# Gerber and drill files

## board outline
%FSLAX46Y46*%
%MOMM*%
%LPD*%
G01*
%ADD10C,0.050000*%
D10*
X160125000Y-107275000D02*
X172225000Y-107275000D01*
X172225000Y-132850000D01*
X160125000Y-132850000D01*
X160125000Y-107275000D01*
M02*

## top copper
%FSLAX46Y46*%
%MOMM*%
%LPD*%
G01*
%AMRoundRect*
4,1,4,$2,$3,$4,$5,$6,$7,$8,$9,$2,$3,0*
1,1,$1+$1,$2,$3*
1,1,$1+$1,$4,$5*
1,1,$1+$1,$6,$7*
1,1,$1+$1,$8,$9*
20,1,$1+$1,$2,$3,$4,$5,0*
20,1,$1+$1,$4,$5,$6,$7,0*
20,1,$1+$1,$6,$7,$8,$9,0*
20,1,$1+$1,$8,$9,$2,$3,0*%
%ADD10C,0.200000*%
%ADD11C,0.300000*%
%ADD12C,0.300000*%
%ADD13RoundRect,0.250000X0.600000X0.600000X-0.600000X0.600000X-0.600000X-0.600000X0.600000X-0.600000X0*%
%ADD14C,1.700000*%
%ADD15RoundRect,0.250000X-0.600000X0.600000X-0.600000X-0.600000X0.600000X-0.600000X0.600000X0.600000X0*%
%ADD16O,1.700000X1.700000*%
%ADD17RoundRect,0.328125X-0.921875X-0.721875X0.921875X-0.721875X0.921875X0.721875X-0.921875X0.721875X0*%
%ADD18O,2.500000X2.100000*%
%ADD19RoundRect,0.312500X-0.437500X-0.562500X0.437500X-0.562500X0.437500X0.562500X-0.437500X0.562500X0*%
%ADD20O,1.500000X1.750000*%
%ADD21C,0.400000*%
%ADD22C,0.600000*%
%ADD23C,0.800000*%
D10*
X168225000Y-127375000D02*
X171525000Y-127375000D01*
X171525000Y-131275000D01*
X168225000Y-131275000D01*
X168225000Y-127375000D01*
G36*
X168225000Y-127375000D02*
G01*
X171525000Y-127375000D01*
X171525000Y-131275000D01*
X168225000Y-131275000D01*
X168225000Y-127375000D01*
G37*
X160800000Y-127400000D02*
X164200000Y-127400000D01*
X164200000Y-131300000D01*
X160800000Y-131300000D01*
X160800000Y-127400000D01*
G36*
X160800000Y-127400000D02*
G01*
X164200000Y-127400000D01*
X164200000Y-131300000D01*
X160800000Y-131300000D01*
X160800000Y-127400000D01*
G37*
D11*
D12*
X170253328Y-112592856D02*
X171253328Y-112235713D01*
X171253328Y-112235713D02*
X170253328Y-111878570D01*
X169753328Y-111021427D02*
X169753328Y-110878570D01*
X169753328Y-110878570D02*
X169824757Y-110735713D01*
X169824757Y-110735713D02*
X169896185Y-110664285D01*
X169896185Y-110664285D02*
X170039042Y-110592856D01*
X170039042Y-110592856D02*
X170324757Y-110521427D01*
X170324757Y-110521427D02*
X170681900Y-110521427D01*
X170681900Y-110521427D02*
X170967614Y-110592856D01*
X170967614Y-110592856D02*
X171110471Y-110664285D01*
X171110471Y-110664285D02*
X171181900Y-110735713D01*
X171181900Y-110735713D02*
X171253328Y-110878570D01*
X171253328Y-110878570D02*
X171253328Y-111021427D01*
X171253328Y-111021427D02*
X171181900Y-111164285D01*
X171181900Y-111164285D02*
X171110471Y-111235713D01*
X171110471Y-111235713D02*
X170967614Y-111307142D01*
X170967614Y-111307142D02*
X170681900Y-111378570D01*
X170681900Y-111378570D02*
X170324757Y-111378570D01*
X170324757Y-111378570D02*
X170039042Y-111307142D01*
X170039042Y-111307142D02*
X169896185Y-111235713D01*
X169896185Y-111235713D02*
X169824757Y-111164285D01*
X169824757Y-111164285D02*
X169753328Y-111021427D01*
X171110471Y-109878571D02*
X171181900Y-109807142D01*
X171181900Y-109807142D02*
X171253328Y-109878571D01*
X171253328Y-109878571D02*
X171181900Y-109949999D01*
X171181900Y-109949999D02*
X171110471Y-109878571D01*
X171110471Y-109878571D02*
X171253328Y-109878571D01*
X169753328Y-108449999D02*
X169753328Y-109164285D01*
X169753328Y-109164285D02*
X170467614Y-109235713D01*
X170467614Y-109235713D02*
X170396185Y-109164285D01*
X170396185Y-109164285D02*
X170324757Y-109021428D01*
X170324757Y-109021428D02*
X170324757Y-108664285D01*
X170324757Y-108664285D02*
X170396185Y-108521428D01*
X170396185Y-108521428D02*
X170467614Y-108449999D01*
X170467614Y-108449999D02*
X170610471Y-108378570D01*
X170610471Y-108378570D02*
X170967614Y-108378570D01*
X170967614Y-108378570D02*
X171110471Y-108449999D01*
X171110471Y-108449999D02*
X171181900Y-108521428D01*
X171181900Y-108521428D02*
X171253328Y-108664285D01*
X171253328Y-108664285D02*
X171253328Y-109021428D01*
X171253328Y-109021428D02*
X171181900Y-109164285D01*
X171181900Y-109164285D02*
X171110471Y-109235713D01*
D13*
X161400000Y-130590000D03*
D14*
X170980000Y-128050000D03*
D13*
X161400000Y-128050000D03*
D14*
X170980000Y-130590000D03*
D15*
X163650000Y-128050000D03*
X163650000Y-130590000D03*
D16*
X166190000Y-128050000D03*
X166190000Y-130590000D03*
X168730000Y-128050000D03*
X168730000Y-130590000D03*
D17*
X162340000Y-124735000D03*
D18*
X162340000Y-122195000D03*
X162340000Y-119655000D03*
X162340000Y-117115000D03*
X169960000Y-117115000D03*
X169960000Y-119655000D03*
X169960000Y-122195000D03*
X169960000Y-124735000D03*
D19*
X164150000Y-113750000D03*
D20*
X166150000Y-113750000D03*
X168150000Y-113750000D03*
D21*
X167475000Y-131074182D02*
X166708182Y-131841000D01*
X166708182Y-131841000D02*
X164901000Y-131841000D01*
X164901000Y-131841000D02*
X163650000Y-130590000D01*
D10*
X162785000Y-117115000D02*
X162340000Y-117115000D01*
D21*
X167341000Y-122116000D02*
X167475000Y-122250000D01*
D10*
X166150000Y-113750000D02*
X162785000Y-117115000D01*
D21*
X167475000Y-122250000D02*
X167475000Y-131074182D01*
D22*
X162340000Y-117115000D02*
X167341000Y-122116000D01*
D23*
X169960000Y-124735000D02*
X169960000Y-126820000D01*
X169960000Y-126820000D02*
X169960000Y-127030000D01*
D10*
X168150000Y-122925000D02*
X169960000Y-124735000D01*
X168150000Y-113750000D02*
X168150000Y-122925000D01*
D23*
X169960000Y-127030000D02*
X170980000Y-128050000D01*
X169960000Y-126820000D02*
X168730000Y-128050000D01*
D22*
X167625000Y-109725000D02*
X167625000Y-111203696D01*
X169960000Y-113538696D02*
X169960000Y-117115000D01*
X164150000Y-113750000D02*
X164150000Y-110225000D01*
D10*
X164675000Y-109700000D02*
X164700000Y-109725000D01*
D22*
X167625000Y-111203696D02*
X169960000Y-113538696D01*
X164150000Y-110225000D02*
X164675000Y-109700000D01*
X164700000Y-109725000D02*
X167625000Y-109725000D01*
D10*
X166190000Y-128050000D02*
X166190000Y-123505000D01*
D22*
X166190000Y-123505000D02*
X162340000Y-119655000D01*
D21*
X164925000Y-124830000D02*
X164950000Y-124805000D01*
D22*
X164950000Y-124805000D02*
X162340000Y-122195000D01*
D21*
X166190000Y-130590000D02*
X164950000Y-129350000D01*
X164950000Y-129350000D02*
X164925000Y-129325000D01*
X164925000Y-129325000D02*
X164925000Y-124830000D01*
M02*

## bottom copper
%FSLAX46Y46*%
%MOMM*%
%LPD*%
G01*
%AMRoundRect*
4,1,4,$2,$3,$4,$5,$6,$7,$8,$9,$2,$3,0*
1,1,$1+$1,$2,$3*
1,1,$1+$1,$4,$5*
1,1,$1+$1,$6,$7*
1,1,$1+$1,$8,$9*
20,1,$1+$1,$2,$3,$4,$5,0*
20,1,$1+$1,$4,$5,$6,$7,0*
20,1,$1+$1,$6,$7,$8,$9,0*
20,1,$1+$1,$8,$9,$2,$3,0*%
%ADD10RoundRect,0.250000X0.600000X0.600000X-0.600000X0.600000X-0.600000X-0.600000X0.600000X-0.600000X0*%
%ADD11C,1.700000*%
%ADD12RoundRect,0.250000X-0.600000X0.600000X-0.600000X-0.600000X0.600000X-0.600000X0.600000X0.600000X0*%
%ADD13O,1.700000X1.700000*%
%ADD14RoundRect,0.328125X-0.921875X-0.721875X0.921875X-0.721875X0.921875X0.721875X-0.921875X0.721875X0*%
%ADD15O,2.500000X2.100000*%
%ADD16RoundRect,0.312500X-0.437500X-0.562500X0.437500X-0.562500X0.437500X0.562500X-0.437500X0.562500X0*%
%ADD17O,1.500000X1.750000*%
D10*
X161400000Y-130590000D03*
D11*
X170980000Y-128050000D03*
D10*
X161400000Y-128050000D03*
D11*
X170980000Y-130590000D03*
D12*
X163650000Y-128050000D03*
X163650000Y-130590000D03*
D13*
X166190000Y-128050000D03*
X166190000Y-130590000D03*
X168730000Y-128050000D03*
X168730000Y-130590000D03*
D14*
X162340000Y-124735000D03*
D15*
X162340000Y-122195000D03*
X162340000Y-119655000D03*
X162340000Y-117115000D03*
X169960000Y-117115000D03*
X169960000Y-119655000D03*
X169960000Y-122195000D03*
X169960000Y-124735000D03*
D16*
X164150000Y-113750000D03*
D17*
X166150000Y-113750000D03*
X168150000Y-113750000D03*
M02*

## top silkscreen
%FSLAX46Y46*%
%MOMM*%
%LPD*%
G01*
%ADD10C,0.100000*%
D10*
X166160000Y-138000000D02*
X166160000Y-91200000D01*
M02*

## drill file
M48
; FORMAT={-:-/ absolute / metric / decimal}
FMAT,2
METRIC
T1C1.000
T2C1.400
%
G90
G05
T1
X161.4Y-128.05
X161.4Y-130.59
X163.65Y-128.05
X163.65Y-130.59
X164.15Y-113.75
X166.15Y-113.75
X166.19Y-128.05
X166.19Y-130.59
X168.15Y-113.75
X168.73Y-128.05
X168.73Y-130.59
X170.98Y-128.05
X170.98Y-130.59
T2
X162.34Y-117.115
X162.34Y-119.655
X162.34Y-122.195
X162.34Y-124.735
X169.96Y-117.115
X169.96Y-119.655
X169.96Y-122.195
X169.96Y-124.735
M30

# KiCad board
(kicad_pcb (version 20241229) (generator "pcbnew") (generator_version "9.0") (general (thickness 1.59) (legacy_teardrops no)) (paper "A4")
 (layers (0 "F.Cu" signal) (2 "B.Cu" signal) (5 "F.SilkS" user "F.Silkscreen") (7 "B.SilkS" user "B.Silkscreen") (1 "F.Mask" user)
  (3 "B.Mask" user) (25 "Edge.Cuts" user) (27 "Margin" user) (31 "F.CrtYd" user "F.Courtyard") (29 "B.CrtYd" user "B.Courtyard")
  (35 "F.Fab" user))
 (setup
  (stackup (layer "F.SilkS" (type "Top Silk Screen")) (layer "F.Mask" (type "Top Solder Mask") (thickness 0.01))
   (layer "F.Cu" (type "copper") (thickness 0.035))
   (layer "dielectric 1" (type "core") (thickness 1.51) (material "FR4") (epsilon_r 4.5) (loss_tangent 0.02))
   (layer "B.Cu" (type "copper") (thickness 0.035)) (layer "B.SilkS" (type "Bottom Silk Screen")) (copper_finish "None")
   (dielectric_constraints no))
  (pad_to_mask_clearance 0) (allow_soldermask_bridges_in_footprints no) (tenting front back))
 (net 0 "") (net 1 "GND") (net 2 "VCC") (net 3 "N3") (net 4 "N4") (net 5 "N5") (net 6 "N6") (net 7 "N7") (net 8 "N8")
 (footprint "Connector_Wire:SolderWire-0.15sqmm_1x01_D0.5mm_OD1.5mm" (layer "F.Cu") (at 161.4 130.59 180)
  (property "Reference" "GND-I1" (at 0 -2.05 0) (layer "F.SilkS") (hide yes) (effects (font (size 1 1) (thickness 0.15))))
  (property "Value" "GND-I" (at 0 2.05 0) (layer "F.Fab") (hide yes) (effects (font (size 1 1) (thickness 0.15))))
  (pad "1" thru_hole roundrect (at 0 0 180) (size 1.7 1.7) (drill 1) (layers "*.Cu" "*.Mask") (remove_unused_layers no)
   (roundrect_rratio 0.147059) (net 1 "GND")))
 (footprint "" (layer "F.Cu") (at 170.98 128.05)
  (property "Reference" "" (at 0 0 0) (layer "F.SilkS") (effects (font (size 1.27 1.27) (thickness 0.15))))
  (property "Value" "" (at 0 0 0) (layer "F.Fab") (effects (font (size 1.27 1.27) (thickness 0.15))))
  (pad "1" thru_hole circle (at 0 0) (size 1.7 1.7) (drill 1) (layers "*.Cu" "*.Mask") (remove_unused_layers no) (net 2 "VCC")))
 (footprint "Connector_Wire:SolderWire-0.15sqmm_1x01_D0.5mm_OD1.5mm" (layer "F.Cu") (at 161.4 128.05 180)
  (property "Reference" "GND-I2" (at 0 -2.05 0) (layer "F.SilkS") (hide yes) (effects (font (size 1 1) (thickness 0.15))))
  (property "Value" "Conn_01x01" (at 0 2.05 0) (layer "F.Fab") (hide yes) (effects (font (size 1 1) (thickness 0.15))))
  (pad "1" thru_hole roundrect (at 0 0 180) (size 1.7 1.7) (drill 1) (layers "*.Cu" "*.Mask") (remove_unused_layers no)
   (roundrect_rratio 0.147059) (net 1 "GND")))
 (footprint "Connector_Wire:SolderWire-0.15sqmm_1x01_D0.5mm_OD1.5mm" (layer "B.Cu") (at 170.98 130.59)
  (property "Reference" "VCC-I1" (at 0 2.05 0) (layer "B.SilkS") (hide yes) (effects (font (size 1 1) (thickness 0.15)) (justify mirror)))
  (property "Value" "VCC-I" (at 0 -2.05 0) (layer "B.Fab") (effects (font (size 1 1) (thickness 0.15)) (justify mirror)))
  (pad "1" thru_hole circle (at 0 0) (size 1.7 1.7) (drill 1) (layers "*.Cu" "*.Mask") (remove_unused_layers no) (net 2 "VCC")))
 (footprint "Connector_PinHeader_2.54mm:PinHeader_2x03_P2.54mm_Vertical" (layer "B.Cu") (at 163.65 128.05 -90)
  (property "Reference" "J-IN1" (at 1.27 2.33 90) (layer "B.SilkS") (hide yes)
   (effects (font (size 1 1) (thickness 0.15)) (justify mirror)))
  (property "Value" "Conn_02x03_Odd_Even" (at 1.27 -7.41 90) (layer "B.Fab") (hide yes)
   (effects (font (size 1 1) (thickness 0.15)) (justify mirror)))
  (pad "1" thru_hole roundrect (at 0 0 270) (size 1.7 1.7) (drill 1) (layers "*.Cu" "*.Mask") (remove_unused_layers no)
   (roundrect_rratio 0.1470588235) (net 1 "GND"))
  (pad "2" thru_hole roundrect (at 2.54 0 270) (size 1.7 1.7) (drill 1) (layers "*.Cu" "*.Mask") (remove_unused_layers no)
   (roundrect_rratio 0.1470588235) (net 1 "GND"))
  (pad "3" thru_hole oval (at 0 -2.54 270) (size 1.7 1.7) (drill 1) (layers "*.Cu" "*.Mask") (remove_unused_layers no) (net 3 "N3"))
  (pad "4" thru_hole oval (at 2.54 -2.54 270) (size 1.7 1.7) (drill 1) (layers "*.Cu" "*.Mask") (remove_unused_layers no) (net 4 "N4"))
  (pad "5" thru_hole oval (at 0 -5.08 270) (size 1.7 1.7) (drill 1) (layers "*.Cu" "*.Mask") (remove_unused_layers no) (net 2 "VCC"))
  (pad "6" thru_hole oval (at 2.54 -5.08 270) (size 1.7 1.7) (drill 1) (layers "*.Cu" "*.Mask") (remove_unused_layers no) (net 2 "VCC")))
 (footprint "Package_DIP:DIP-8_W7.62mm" (layer "B.Cu") (at 162.34 124.735)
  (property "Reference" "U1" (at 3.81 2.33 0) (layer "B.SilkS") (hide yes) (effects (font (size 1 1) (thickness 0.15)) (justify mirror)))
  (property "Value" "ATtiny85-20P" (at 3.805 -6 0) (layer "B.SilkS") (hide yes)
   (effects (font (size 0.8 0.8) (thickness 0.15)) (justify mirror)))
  (pad "1" thru_hole roundrect (at 0 0) (size 2.5 2.1) (drill 1.4) (layers "*.Cu" "*.Mask") (remove_unused_layers no)
   (roundrect_rratio 0.15625) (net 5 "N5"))
  (pad "2" thru_hole oval (at 0 -2.54) (size 2.5 2.1) (drill 1.4) (layers "*.Cu" "*.Mask") (remove_unused_layers no) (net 4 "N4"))
  (pad "3" thru_hole oval (at 0 -5.08) (size 2.5 2.1) (drill 1.4) (layers "*.Cu" "*.Mask") (remove_unused_layers no) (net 3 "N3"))
  (pad "4" thru_hole oval (at 0 -7.62) (size 2.5 2.1) (drill 1.4) (layers "*.Cu" "*.Mask") (remove_unused_layers no) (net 1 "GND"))
  (pad "5" thru_hole oval (at 7.62 -7.62) (size 2.5 2.1) (drill 1.4) (layers "*.Cu" "*.Mask") (remove_unused_layers no) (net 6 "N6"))
  (pad "6" thru_hole oval (at 7.62 -5.08) (size 2.5 2.1) (drill 1.4) (layers "*.Cu" "*.Mask") (remove_unused_layers no) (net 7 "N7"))
  (pad "7" thru_hole oval (at 7.62 -2.54) (size 2.5 2.1) (drill 1.4) (layers "*.Cu" "*.Mask") (remove_unused_layers no) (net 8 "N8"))
  (pad "8" thru_hole oval (at 7.62 0) (size 2.5 2.1) (drill 1.4) (layers "*.Cu" "*.Mask") (remove_unused_layers no) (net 2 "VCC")))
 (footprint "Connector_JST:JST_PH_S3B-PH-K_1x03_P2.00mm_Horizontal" (layer "B.Cu") (at 164.15 113.75)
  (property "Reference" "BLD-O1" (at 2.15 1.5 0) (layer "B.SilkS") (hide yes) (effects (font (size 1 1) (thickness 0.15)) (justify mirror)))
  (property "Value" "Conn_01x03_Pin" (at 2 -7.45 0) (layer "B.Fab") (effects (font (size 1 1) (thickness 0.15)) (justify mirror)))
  (pad "1" thru_hole roundrect (at 0 0) (size 1.5 1.75) (drill 1) (layers "*.Cu" "*.Mask") (remove_unused_layers no)
   (roundrect_rratio 0.208333) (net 6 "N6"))
  (pad "2" thru_hole oval (at 2 0) (size 1.5 1.75) (drill 1) (layers "*.Cu" "*.Mask") (remove_unused_layers no) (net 1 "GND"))
  (pad "3" thru_hole oval (at 4 0) (size 1.5 1.75) (drill 1) (layers "*.Cu" "*.Mask") (remove_unused_layers no) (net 2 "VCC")))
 (gr_rect (start 168.225 127.375) (end 171.525 131.275) (stroke (width 0.2) (type solid)) (fill yes) (layer "F.Cu") (net 2))
 (gr_rect (start 160.8 127.4) (end 164.2 131.3) (stroke (width 0.2) (type solid)) (fill yes) (layer "F.Cu") (net 1))
 (gr_line (start 166.16 138) (end 166.16 91.2) (stroke (width 0.1) (type default)) (layer "F.SilkS"))
 (gr_rect (start 160.125 107.275) (end 172.225 132.85) (stroke (width 0.05) (type solid)) (fill no) (layer "Edge.Cuts"))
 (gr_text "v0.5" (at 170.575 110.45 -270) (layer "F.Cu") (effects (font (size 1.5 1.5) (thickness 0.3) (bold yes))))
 (segment (start 167.475 131.074182) (end 166.708182 131.841) (width 0.4) (layer "F.Cu") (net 1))
 (segment (start 166.708182 131.841) (end 164.901 131.841) (width 0.4) (layer "F.Cu") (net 1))
 (segment (start 164.901 131.841) (end 163.65 130.59) (width 0.4) (layer "F.Cu") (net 1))
 (segment (start 162.785 117.115) (end 162.34 117.115) (width 0.2) (layer "F.Cu") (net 1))
 (segment (start 167.341 122.116) (end 167.475 122.25) (width 0.4) (layer "F.Cu") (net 1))
 (segment (start 166.15 113.75) (end 162.785 117.115) (width 0.2) (layer "F.Cu") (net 1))
 (segment (start 167.475 122.25) (end 167.475 131.074182) (width 0.4) (layer "F.Cu") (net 1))
 (segment (start 162.34 117.115) (end 167.341 122.116) (width 0.6) (layer "F.Cu") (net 1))
 (segment (start 169.96 124.735) (end 169.96 126.82) (width 0.8) (layer "F.Cu") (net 2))
 (segment (start 169.96 126.82) (end 169.96 127.03) (width 0.8) (layer "F.Cu") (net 2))
 (segment (start 168.15 122.925) (end 169.96 124.735) (width 0.2) (layer "F.Cu") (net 2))
 (segment (start 168.15 113.75) (end 168.15 122.925) (width 0.2) (layer "F.Cu") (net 2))
 (segment (start 169.96 127.03) (end 170.98 128.05) (width 0.8) (layer "F.Cu") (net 2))
 (segment (start 169.96 126.82) (end 168.73 128.05) (width 0.8) (layer "F.Cu") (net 2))
 (segment (start 167.625 109.725) (end 167.625 111.203696) (width 0.6) (layer "F.Cu") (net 6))
 (segment (start 169.96 113.538696) (end 169.96 117.115) (width 0.6) (layer "F.Cu") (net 6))
 (segment (start 164.15 113.75) (end 164.15 110.225) (width 0.6) (layer "F.Cu") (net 6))
 (segment (start 164.675 109.7) (end 164.7 109.725) (width 0.2) (layer "F.Cu") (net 6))
 (segment (start 167.625 111.203696) (end 169.96 113.538696) (width 0.6) (layer "F.Cu") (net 6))
 (segment (start 164.15 110.225) (end 164.675 109.7) (width 0.6) (layer "F.Cu") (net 6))
 (segment (start 164.7 109.725) (end 167.625 109.725) (width 0.6) (layer "F.Cu") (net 6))
 (segment (start 166.19 128.05) (end 166.19 123.505) (width 0.2) (layer "F.Cu") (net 3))
 (segment (start 166.19 123.505) (end 162.34 119.655) (width 0.6) (layer "F.Cu") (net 3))
 (segment (start 164.925 124.83) (end 164.95 124.805) (width 0.4) (layer "F.Cu") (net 4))
 (segment (start 164.95 124.805) (end 162.34 122.195) (width 0.6) (layer "F.Cu") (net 4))
 (segment (start 166.19 130.59) (end 164.95 129.35) (width 0.4) (layer "F.Cu") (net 4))
 (segment (start 164.95 129.35) (end 164.925 129.325) (width 0.4) (layer "F.Cu") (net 4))
 (segment (start 164.925 129.325) (end 164.925 124.83) (width 0.4) (layer "F.Cu") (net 4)))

